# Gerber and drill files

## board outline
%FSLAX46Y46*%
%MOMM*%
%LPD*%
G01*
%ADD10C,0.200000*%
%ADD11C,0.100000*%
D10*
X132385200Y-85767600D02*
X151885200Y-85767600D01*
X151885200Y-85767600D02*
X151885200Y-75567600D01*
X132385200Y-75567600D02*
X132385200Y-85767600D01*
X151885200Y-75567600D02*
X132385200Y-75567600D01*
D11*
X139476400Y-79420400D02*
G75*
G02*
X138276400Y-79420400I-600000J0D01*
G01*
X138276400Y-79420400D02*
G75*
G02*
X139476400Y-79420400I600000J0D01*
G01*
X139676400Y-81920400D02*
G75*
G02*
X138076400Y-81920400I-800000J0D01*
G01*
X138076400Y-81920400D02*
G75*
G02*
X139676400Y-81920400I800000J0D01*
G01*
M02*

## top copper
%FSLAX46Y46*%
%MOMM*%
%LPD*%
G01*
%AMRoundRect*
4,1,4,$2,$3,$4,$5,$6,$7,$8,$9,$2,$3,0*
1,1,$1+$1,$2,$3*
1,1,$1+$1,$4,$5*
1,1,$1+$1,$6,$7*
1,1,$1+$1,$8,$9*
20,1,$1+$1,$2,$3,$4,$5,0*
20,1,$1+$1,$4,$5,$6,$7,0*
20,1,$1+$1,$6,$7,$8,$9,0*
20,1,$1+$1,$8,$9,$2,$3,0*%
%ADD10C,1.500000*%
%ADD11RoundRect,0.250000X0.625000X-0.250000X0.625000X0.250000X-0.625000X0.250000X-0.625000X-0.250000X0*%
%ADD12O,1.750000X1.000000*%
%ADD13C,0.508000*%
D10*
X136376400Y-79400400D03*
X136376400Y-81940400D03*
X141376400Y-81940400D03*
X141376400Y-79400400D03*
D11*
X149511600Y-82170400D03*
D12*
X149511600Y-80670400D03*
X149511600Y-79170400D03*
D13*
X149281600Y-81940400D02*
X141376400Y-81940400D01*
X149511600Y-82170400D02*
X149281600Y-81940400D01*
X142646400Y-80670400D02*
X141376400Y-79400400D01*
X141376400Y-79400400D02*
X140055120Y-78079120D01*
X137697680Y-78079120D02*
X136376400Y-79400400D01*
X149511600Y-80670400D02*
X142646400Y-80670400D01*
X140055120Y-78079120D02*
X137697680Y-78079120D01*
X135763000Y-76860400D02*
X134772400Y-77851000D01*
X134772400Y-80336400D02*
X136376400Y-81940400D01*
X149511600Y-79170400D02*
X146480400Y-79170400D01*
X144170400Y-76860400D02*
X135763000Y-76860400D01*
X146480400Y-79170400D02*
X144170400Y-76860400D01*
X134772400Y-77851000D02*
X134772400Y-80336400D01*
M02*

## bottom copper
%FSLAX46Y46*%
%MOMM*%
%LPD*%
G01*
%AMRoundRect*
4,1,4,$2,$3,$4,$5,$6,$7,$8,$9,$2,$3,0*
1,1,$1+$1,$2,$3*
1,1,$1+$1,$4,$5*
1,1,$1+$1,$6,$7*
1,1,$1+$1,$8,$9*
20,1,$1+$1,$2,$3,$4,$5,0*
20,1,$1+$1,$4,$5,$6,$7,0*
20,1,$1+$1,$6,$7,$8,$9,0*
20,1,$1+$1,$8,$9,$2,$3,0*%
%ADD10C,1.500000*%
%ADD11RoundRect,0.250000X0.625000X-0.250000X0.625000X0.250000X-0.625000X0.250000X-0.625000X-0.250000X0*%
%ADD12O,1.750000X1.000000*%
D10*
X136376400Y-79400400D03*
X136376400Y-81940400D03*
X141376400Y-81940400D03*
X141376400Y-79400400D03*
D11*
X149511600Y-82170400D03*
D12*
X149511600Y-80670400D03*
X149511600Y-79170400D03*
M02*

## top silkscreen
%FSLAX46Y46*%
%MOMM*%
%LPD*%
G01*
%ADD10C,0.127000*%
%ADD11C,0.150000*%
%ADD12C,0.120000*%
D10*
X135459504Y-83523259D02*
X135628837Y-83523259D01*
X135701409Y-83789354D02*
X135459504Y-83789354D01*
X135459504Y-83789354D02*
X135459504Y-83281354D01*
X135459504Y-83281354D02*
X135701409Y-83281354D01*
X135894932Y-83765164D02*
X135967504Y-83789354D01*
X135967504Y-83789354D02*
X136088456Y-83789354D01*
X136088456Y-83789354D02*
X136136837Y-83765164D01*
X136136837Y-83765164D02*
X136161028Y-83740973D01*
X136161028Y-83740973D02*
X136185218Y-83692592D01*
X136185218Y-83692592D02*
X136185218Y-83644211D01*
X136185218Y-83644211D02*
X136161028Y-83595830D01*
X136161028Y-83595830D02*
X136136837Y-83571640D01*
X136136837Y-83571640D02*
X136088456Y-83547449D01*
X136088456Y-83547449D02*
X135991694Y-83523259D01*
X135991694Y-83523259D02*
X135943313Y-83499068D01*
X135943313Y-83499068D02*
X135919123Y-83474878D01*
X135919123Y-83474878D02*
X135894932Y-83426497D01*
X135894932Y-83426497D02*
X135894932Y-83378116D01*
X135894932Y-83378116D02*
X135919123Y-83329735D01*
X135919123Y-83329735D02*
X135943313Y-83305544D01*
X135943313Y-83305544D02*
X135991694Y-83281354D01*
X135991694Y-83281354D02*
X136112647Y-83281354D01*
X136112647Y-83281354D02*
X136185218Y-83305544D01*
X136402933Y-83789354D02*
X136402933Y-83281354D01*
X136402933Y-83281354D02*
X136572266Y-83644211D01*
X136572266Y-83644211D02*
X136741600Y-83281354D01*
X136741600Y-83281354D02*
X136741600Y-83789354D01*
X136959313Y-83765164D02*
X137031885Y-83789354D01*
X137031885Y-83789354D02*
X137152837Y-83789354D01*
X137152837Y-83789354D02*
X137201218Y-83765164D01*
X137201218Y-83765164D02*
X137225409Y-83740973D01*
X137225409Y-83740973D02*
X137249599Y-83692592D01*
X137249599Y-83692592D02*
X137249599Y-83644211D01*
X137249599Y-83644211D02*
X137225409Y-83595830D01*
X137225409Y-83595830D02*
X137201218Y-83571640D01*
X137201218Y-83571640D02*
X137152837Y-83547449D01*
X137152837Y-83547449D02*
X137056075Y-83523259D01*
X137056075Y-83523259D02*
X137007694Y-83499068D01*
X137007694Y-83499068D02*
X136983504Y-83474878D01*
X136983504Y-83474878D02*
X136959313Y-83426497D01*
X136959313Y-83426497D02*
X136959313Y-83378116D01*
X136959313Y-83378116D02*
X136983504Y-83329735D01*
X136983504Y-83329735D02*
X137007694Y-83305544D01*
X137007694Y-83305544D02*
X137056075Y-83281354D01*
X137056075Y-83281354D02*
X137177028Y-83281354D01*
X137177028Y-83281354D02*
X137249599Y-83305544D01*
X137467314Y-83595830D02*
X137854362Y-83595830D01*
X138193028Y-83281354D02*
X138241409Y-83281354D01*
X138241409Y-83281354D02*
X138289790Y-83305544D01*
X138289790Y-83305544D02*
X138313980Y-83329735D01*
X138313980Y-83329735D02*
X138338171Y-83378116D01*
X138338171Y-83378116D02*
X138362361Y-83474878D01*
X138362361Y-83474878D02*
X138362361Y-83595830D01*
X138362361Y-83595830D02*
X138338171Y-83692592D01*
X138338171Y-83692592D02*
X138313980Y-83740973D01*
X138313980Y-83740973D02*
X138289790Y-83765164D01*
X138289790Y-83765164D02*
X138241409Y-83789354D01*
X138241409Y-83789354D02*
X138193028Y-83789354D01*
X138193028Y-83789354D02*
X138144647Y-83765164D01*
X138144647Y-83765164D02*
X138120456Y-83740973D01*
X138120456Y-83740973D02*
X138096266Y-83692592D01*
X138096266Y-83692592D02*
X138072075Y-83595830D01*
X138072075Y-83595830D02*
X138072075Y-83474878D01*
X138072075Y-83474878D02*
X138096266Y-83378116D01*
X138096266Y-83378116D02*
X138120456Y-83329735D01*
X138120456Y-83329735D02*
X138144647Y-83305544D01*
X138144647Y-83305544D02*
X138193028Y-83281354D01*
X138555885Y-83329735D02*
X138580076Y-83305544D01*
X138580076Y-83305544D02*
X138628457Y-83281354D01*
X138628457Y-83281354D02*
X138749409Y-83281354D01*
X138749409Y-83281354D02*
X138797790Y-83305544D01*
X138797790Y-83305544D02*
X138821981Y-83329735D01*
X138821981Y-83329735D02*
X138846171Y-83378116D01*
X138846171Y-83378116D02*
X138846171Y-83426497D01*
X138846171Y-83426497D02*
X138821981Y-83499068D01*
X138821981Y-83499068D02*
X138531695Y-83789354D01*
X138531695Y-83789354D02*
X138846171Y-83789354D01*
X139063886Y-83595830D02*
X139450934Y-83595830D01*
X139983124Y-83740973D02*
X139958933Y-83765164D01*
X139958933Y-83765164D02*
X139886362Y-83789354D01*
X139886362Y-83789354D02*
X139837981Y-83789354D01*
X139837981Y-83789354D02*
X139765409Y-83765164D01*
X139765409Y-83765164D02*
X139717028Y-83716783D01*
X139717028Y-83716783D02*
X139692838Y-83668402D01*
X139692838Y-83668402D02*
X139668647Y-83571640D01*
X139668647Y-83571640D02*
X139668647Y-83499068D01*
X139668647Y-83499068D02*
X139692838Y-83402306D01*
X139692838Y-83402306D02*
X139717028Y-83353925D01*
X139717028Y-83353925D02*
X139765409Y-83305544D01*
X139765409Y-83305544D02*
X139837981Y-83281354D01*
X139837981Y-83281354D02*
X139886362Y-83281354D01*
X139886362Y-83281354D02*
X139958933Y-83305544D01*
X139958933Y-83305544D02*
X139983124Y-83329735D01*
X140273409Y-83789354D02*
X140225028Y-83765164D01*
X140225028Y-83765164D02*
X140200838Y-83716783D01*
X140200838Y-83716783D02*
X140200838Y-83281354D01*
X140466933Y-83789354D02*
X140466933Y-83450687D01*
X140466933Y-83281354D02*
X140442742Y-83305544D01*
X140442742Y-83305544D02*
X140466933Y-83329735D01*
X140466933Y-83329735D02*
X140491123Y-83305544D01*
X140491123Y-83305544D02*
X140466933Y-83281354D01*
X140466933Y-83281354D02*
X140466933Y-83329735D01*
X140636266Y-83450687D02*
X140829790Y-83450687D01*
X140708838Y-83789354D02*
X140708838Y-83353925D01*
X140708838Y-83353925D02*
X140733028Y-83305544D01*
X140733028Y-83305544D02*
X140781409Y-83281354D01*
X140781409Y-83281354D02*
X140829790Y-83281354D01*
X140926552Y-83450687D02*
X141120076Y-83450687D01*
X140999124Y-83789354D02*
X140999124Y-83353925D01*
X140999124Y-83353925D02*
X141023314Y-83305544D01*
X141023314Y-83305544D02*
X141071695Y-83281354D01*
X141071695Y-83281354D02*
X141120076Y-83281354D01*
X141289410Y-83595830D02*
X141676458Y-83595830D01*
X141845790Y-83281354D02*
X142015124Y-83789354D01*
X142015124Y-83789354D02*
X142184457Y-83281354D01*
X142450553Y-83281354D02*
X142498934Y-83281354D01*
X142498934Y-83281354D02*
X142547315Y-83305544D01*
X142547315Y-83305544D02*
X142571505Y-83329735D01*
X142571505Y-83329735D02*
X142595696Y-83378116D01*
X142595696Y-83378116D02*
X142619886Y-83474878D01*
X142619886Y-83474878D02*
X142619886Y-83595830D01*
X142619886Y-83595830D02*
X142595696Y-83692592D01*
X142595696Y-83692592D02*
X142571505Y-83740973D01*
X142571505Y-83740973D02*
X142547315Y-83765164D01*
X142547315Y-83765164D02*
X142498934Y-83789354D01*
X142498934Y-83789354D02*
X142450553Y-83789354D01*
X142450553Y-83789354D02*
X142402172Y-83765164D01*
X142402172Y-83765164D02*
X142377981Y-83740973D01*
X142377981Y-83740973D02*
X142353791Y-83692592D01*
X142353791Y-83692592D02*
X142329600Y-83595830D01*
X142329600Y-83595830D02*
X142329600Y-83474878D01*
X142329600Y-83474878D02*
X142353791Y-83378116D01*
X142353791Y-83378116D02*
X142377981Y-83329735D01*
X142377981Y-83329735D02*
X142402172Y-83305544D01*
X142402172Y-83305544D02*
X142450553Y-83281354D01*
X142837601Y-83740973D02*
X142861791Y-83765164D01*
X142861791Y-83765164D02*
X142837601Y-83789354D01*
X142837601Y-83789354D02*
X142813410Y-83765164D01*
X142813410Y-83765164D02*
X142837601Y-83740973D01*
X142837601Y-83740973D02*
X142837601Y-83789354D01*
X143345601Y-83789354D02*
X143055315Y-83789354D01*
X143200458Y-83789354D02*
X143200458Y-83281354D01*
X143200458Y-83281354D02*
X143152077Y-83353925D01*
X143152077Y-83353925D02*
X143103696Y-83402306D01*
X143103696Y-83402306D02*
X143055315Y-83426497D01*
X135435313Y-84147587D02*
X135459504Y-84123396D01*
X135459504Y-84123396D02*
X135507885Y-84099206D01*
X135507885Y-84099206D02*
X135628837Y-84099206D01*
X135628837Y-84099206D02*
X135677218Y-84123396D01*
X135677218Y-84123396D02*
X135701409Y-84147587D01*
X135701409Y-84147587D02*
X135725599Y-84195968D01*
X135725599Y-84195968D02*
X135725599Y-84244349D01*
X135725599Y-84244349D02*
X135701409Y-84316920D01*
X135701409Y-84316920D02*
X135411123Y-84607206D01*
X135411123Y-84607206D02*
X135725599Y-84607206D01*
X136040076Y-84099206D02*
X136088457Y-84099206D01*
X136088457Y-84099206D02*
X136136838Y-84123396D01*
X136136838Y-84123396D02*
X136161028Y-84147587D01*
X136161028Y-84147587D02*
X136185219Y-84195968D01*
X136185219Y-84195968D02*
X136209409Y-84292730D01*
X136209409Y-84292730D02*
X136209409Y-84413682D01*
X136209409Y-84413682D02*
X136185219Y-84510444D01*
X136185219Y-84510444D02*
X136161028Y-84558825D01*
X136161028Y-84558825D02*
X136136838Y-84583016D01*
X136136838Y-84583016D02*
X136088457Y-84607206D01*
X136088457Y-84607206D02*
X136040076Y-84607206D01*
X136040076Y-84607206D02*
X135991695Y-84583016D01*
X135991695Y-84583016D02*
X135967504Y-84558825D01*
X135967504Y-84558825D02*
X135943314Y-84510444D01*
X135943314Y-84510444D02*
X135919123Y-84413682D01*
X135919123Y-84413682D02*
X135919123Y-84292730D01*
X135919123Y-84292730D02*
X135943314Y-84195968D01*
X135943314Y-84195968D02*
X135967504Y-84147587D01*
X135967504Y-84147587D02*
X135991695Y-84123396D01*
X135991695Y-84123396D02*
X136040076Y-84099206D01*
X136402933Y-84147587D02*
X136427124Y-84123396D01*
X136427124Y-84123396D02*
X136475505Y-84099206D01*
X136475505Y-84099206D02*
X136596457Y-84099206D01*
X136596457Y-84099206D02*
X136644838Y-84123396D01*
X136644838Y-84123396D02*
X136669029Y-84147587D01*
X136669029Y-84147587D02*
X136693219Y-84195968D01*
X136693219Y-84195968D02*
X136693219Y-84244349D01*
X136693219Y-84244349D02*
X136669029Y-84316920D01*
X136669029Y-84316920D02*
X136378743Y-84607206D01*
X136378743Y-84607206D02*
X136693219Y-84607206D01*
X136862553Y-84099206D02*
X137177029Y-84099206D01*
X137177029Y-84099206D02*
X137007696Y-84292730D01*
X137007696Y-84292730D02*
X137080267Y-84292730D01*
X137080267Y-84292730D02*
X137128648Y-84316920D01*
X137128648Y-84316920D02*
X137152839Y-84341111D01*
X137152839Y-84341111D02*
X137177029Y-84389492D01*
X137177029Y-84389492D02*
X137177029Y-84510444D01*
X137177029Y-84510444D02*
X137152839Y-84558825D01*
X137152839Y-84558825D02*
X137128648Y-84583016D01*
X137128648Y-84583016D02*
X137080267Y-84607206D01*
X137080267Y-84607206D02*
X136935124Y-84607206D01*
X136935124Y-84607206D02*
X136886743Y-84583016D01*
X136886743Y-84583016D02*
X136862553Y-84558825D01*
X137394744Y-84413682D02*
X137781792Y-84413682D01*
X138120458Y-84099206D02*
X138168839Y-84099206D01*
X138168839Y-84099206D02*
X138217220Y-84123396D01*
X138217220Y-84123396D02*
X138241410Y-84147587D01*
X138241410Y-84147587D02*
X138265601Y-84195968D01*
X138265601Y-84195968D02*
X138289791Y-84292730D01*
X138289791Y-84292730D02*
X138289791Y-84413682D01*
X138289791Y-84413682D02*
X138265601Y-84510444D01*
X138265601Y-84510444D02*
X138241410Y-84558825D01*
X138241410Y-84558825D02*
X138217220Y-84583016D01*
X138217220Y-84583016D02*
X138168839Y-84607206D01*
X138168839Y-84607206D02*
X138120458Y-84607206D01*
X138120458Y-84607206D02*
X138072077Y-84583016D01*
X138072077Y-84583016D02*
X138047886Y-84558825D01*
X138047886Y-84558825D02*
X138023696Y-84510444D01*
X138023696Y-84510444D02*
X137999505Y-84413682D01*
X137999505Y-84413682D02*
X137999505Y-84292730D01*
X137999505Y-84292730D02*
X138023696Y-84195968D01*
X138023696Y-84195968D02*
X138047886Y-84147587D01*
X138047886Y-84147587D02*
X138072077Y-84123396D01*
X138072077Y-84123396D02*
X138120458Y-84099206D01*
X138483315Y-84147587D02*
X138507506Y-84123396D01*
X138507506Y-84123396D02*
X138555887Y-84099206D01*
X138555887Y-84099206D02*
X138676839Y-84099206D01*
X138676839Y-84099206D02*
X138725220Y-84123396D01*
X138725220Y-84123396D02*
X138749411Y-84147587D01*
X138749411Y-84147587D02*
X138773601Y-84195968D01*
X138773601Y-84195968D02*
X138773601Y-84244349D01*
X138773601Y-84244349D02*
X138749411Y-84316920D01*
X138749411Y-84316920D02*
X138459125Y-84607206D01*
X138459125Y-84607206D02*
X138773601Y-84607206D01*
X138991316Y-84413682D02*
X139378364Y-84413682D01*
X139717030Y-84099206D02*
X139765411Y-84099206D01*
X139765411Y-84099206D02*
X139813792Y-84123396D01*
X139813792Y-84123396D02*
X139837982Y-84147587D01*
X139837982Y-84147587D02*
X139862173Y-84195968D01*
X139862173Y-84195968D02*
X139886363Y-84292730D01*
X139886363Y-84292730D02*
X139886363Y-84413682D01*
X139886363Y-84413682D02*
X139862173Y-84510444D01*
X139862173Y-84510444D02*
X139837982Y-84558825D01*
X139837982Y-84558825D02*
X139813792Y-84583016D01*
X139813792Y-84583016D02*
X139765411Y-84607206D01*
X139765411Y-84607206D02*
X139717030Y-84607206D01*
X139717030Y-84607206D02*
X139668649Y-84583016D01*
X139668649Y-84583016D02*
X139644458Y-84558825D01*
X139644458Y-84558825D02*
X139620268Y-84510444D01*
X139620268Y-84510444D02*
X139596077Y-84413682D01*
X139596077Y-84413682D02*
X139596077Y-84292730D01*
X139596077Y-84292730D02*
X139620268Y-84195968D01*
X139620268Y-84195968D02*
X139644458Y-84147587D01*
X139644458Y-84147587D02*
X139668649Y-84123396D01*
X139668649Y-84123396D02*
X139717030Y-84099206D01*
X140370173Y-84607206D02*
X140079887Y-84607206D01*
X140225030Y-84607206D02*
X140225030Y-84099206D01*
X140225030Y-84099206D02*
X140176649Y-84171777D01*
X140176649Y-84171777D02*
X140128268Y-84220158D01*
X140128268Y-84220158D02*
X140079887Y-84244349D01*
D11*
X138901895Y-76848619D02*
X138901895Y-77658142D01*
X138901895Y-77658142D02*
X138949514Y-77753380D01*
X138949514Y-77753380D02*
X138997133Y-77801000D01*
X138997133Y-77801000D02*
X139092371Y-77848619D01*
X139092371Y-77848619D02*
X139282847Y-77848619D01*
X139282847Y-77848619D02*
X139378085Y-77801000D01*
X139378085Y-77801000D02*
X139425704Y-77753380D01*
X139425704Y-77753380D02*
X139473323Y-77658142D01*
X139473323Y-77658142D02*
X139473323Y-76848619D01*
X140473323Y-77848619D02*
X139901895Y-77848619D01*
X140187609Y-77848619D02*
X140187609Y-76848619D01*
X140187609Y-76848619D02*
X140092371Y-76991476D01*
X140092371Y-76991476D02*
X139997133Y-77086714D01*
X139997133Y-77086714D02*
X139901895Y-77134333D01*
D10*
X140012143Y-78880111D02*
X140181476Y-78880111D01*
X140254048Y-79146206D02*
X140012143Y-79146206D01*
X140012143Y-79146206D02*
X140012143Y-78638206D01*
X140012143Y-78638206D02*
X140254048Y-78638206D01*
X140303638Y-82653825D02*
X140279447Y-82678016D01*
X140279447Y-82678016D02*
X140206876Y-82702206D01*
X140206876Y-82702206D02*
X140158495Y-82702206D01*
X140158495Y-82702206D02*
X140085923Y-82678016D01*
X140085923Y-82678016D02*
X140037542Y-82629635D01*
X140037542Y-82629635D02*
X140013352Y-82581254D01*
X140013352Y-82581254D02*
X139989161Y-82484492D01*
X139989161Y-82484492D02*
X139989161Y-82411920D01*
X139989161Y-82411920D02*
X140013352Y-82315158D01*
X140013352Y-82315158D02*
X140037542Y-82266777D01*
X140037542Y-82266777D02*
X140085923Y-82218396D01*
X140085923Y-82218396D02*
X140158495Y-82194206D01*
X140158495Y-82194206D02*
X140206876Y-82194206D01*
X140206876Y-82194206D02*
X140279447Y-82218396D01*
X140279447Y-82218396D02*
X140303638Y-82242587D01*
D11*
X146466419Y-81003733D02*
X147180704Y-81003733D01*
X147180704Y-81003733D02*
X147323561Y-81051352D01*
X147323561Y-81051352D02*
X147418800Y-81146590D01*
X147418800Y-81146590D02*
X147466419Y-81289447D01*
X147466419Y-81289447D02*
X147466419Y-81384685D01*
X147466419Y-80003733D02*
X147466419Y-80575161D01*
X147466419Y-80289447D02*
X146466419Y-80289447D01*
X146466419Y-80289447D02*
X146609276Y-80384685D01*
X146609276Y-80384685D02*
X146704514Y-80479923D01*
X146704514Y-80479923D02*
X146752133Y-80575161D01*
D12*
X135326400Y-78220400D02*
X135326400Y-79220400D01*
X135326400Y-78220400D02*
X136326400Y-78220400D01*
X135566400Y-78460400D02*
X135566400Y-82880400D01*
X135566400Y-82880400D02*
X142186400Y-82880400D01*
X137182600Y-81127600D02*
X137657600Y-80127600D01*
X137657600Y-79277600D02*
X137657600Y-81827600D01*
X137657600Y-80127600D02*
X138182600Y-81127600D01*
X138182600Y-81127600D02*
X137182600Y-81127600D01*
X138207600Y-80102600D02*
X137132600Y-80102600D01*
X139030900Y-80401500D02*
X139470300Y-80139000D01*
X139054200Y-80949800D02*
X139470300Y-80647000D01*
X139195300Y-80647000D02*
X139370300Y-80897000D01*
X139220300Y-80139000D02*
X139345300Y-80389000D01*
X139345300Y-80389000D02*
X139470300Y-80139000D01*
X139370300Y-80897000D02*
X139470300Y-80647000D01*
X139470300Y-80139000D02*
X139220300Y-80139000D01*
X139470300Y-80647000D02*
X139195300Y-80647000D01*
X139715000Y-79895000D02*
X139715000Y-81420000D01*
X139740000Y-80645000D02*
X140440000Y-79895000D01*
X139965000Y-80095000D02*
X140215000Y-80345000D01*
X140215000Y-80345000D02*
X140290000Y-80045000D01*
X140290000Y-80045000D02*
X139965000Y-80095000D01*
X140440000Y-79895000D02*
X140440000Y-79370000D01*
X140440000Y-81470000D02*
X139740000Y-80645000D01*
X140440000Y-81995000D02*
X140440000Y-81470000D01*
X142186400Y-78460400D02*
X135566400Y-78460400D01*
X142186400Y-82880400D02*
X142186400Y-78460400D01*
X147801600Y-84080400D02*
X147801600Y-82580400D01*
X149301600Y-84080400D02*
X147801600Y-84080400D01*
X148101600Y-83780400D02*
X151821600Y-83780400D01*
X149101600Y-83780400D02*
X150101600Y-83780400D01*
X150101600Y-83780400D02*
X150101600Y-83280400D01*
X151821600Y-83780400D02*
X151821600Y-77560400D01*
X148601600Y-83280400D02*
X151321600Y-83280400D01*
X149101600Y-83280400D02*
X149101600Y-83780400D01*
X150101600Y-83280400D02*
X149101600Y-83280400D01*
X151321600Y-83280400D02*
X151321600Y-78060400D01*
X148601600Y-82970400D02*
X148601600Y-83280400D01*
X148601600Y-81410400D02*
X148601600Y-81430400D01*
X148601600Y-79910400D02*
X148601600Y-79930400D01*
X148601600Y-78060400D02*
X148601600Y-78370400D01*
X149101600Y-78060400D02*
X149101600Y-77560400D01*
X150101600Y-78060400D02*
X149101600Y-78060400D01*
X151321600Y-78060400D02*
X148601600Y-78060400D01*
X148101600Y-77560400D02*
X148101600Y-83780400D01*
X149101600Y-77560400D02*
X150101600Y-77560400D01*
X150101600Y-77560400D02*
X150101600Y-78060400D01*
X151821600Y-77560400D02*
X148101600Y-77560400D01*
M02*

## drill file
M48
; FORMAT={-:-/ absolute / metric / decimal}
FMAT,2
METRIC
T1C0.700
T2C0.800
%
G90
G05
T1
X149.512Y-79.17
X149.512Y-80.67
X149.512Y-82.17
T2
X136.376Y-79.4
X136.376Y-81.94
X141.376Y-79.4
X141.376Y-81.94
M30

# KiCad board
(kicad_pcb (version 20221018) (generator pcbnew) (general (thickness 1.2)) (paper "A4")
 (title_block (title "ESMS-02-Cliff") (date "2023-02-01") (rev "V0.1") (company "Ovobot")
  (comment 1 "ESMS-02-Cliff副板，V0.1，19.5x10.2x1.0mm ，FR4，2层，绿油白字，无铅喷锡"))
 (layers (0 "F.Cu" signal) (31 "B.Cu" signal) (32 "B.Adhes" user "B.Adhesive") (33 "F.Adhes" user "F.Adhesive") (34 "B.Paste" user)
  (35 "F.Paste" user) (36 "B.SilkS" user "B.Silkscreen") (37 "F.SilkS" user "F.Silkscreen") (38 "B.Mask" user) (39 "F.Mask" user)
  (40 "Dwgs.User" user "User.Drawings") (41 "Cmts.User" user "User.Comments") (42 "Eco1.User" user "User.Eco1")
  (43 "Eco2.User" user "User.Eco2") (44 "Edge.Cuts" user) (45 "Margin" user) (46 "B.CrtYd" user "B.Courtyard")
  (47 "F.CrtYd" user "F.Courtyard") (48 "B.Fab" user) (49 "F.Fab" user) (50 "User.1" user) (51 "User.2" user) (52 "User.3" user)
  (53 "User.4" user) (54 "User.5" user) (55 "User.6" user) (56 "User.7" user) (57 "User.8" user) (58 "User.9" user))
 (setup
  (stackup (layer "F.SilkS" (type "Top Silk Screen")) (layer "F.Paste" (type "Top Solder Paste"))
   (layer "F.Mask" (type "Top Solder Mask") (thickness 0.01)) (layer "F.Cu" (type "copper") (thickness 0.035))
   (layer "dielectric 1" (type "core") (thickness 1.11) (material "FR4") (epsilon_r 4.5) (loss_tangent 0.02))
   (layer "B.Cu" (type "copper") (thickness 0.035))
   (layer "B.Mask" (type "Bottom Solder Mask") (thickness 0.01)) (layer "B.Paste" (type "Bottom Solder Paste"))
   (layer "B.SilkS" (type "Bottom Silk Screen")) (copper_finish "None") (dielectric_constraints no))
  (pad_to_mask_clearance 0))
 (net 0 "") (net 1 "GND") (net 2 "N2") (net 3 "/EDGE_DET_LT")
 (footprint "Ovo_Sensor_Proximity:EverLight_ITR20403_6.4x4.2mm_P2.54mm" (layer "F.Cu") (at 138.8764 80.6704)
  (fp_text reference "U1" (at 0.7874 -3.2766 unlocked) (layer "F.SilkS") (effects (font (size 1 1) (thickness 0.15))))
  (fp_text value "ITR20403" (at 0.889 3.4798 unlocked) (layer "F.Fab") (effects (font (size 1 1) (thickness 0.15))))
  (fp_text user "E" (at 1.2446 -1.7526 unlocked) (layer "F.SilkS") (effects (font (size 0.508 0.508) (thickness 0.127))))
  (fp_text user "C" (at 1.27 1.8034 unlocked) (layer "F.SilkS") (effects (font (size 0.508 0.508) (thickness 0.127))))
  (fp_line (start -3.55 -2.45) (end -3.55 -1.45) (stroke (width 0.12) (type solid)) (layer "F.SilkS"))
  (fp_line (start -3.55 -2.45) (end -2.55 -2.45) (stroke (width 0.12) (type solid)) (layer "F.SilkS"))
  (fp_line (start -3.31 -2.21) (end -3.31 2.21) (stroke (width 0.12) (type solid)) (layer "F.SilkS"))
  (fp_line (start -3.31 2.21) (end 3.31 2.21) (stroke (width 0.12) (type solid)) (layer "F.SilkS"))
  (fp_line (start -1.6938 0.4572) (end -1.2188 -0.5428) (stroke (width 0.12) (type solid)) (layer "F.SilkS"))
  (fp_line (start -1.2188 -1.3928) (end -1.2188 1.1572) (stroke (width 0.12) (type solid)) (layer "F.SilkS"))
  (fp_line (start -1.2188 -0.5428) (end -0.6938 0.4572) (stroke (width 0.12) (type solid)) (layer "F.SilkS"))
  (fp_line (start -0.6938 0.4572) (end -1.6938 0.4572) (stroke (width 0.12) (type solid)) (layer "F.SilkS"))
  (fp_line (start -0.6688 -0.5678) (end -1.7438 -0.5678) (stroke (width 0.12) (type solid)) (layer "F.SilkS"))
  (fp_line (start 0.1545 -0.2689) (end 0.5939 -0.5314) (stroke (width 0.12) (type solid)) (layer "F.SilkS"))
  (fp_line (start 0.1778 0.2794) (end 0.5939 -0.0234) (stroke (width 0.12) (type solid)) (layer "F.SilkS"))
  (fp_line (start 0.3189 -0.0234) (end 0.4939 0.2266) (stroke (width 0.12) (type solid)) (layer "F.SilkS"))
  (fp_line (start 0.3439 -0.5314) (end 0.4689 -0.2814) (stroke (width 0.12) (type solid)) (layer "F.SilkS"))
  (fp_line (start 0.4689 -0.2814) (end 0.5939 -0.5314) (stroke (width 0.12) (type solid)) (layer "F.SilkS"))
  (fp_line (start 0.4939 0.2266) (end 0.5939 -0.0234) (stroke (width 0.12) (type solid)) (layer "F.SilkS"))
  (fp_line (start 0.5939 -0.5314) (end 0.3439 -0.5314) (stroke (width 0.12) (type solid)) (layer "F.SilkS"))
  (fp_line (start 0.5939 -0.0234) (end 0.3189 -0.0234) (stroke (width 0.12) (type solid)) (layer "F.SilkS"))
  (fp_line (start 0.8386 -0.7754) (end 0.8386 0.7496) (stroke (width 0.12) (type solid)) (layer "F.SilkS"))
  (fp_line (start 0.8636 -0.0254) (end 1.5636 -0.7754) (stroke (width 0.12) (type solid)) (layer "F.SilkS"))
  (fp_line (start 1.0886 -0.5754) (end 1.3386 -0.3254) (stroke (width 0.12) (type solid)) (layer "F.SilkS"))
  (fp_line (start 1.3386 -0.3254) (end 1.4136 -0.6254) (stroke (width 0.12) (type solid)) (layer "F.SilkS"))
  (fp_line (start 1.4136 -0.6254) (end 1.0886 -0.5754) (stroke (width 0.12) (type solid)) (layer "F.SilkS"))
  (fp_line (start 1.5636 -0.7754) (end 1.5636 -1.3004) (stroke (width 0.12) (type solid)) (layer "F.SilkS"))
  (fp_line (start 1.5636 0.7996) (end 0.8636 -0.0254) (stroke (width 0.12) (type solid)) (layer "F.SilkS"))
  (fp_line (start 1.5636 1.3246) (end 1.5636 0.7996) (stroke (width 0.12) (type solid)) (layer "F.SilkS"))
  (fp_line (start 3.31 -2.21) (end -3.31 -2.21) (stroke (width 0.12) (type solid)) (layer "F.SilkS"))
  (fp_line (start 3.31 2.21) (end 3.31 -2.21) (stroke (width 0.12) (type solid)) (layer "F.SilkS"))
  (fp_circle (center 0 -1.25) (end 0.6 -1.25) (stroke (width 0.1) (type solid)) (fill none) (layer "Edge.Cuts"))
  (fp_circle (center 0 1.25) (end 0.8 1.25) (stroke (width 0.1) (type solid)) (fill none) (layer "Edge.Cuts"))
  (pad "1" thru_hole circle (at -2.5 -1.27) (size 1.5 1.5) (drill 0.8) (layers "*.Cu" "*.Mask") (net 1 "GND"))
  (pad "2" thru_hole circle (at -2.5 1.27) (size 1.5 1.5) (drill 0.8) (layers "*.Cu" "*.Mask") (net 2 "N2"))
  (pad "3" thru_hole circle (at 2.5 1.27) (size 1.5 1.5) (drill 0.8) (layers "*.Cu" "*.Mask") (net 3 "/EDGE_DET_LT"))
  (pad "4" thru_hole circle (at 2.5 -1.27) (size 1.5 1.5) (drill 0.8) (layers "*.Cu" "*.Mask") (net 1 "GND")))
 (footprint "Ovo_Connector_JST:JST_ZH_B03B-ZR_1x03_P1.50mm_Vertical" (layer "F.Cu") (at 149.5116 82.1704 90)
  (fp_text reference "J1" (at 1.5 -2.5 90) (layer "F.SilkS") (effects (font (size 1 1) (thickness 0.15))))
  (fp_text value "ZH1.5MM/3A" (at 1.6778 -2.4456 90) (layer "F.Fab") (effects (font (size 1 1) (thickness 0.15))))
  (fp_line (start -1.91 -1.71) (end -0.41 -1.71) (stroke (width 0.12) (type solid)) (layer "F.SilkS"))
  (fp_line (start -1.91 -0.21) (end -1.91 -1.71) (stroke (width 0.12) (type solid)) (layer "F.SilkS"))
  (fp_line (start -1.61 -1.41) (end -1.61 2.31) (stroke (width 0.12) (type solid)) (layer "F.SilkS"))
  (fp_line (start -1.61 -0.41) (end -1.61 0.59) (stroke (width 0.12) (type solid)) (layer "F.SilkS"))
  (fp_line (start -1.61 0.59) (end -1.11 0.59) (stroke (width 0.12) (type solid)) (layer "F.SilkS"))
  (fp_line (start -1.61 2.31) (end 4.61 2.31) (stroke (width 0.12) (type solid)) (layer "F.SilkS"))
  (fp_line (start -1.11 -0.91) (end -1.11 1.81) (stroke (width 0.12) (type solid)) (layer "F.SilkS"))
  (fp_line (start -1.11 -0.41) (end -1.61 -0.41) (stroke (width 0.12) (type solid)) (layer "F.SilkS"))
  (fp_line (start -1.11 0.59) (end -1.11 -0.41) (stroke (width 0.12) (type solid)) (layer "F.SilkS"))
  (fp_line (start -1.11 1.81) (end 4.11 1.81) (stroke (width 0.12) (type solid)) (layer "F.SilkS"))
  (fp_line (start -0.8 -0.91) (end -1.11 -0.91) (stroke (width 0.12) (type solid)) (layer "F.SilkS"))
  (fp_line (start 0.76 -0.91) (end 0.74 -0.91) (stroke (width 0.12) (type solid)) (layer "F.SilkS"))
  (fp_line (start 2.26 -0.91) (end 2.24 -0.91) (stroke (width 0.12) (type solid)) (layer "F.SilkS"))
  (fp_line (start 4.11 -0.91) (end 3.8 -0.91) (stroke (width 0.12) (type solid)) (layer "F.SilkS"))
  (fp_line (start 4.11 -0.41) (end 4.61 -0.41) (stroke (width 0.12) (type solid)) (layer "F.SilkS"))
  (fp_line (start 4.11 0.59) (end 4.11 -0.41) (stroke (width 0.12) (type solid)) (layer "F.SilkS"))
  (fp_line (start 4.11 1.81) (end 4.11 -0.91) (stroke (width 0.12) (type solid)) (layer "F.SilkS"))
  (fp_line (start 4.61 -1.41) (end -1.61 -1.41) (stroke (width 0.12) (type solid)) (layer "F.SilkS"))
  (fp_line (start 4.61 -0.41) (end 4.61 0.59) (stroke (width 0.12) (type solid)) (layer "F.SilkS"))
  (fp_line (start 4.61 0.59) (end 4.11 0.59) (stroke (width 0.12) (type solid)) (layer "F.SilkS"))
  (fp_line (start 4.61 2.31) (end 4.61 -1.41) (stroke (width 0.12) (type solid)) (layer "F.SilkS"))
  (pad "1" thru_hole roundrect (at 0 0 90) (size 1 1.75) (drill 0.7) (layers "*.Cu" "*.Mask") (roundrect_rratio 0.25) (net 3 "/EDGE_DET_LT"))
  (pad "2" thru_hole oval (at 1.5 0 90) (size 1 1.75) (drill 0.7) (layers "*.Cu" "*.Mask") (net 1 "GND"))
  (pad "3" thru_hole oval (at 3 0 90) (size 1 1.75) (drill 0.7) (layers "*.Cu" "*.Mask") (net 2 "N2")))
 (gr_line (start 132.3852 85.7676) (end 151.8852 85.7676) (stroke (width 0.2) (type solid)) (layer "Edge.Cuts"))
 (gr_line (start 151.8852 85.7676) (end 151.8852 75.5676) (stroke (width 0.2) (type solid)) (layer "Edge.Cuts"))
 (gr_line (start 132.3852 75.5676) (end 132.3852 85.7676) (stroke (width 0.2) (type solid)) (layer "Edge.Cuts"))
 (gr_line (start 151.8852 75.5676) (end 132.3852 75.5676) (stroke (width 0.2) (type solid)) (layer "Edge.Cuts"))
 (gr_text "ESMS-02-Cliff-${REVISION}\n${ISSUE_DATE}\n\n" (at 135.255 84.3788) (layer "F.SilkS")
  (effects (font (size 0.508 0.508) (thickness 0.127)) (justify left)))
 (segment (start 149.2816 81.9404) (end 141.3764 81.9404) (width 0.508) (layer "F.Cu") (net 3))
 (segment (start 149.5116 82.1704) (end 149.2816 81.9404) (width 0.508) (layer "F.Cu") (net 3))
 (segment (start 142.6464 80.6704) (end 141.3764 79.4004) (width 0.508) (layer "F.Cu") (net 1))
 (segment (start 141.3764 79.4004) (end 140.05512 78.07912) (width 0.508) (layer "F.Cu") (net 1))
 (segment (start 137.69768 78.07912) (end 136.3764 79.4004) (width 0.508) (layer "F.Cu") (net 1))
 (segment (start 149.5116 80.6704) (end 142.6464 80.6704) (width 0.508) (layer "F.Cu") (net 1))
 (segment (start 140.05512 78.07912) (end 137.69768 78.07912) (width 0.508) (layer "F.Cu") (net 1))
 (segment (start 135.763 76.8604) (end 134.7724 77.851) (width 0.508) (layer "F.Cu") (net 2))
 (segment (start 134.7724 80.3364) (end 136.3764 81.9404) (width 0.508) (layer "F.Cu") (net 2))
 (segment (start 149.5116 79.1704) (end 146.4804 79.1704) (width 0.508) (layer "F.Cu") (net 2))
 (segment (start 144.1704 76.8604) (end 135.763 76.8604) (width 0.508) (layer "F.Cu") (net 2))
 (segment (start 146.4804 79.1704) (end 144.1704 76.8604) (width 0.508) (layer "F.Cu") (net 2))
 (segment (start 134.7724 77.851) (end 134.7724 80.3364) (width 0.508) (layer "F.Cu") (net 2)))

